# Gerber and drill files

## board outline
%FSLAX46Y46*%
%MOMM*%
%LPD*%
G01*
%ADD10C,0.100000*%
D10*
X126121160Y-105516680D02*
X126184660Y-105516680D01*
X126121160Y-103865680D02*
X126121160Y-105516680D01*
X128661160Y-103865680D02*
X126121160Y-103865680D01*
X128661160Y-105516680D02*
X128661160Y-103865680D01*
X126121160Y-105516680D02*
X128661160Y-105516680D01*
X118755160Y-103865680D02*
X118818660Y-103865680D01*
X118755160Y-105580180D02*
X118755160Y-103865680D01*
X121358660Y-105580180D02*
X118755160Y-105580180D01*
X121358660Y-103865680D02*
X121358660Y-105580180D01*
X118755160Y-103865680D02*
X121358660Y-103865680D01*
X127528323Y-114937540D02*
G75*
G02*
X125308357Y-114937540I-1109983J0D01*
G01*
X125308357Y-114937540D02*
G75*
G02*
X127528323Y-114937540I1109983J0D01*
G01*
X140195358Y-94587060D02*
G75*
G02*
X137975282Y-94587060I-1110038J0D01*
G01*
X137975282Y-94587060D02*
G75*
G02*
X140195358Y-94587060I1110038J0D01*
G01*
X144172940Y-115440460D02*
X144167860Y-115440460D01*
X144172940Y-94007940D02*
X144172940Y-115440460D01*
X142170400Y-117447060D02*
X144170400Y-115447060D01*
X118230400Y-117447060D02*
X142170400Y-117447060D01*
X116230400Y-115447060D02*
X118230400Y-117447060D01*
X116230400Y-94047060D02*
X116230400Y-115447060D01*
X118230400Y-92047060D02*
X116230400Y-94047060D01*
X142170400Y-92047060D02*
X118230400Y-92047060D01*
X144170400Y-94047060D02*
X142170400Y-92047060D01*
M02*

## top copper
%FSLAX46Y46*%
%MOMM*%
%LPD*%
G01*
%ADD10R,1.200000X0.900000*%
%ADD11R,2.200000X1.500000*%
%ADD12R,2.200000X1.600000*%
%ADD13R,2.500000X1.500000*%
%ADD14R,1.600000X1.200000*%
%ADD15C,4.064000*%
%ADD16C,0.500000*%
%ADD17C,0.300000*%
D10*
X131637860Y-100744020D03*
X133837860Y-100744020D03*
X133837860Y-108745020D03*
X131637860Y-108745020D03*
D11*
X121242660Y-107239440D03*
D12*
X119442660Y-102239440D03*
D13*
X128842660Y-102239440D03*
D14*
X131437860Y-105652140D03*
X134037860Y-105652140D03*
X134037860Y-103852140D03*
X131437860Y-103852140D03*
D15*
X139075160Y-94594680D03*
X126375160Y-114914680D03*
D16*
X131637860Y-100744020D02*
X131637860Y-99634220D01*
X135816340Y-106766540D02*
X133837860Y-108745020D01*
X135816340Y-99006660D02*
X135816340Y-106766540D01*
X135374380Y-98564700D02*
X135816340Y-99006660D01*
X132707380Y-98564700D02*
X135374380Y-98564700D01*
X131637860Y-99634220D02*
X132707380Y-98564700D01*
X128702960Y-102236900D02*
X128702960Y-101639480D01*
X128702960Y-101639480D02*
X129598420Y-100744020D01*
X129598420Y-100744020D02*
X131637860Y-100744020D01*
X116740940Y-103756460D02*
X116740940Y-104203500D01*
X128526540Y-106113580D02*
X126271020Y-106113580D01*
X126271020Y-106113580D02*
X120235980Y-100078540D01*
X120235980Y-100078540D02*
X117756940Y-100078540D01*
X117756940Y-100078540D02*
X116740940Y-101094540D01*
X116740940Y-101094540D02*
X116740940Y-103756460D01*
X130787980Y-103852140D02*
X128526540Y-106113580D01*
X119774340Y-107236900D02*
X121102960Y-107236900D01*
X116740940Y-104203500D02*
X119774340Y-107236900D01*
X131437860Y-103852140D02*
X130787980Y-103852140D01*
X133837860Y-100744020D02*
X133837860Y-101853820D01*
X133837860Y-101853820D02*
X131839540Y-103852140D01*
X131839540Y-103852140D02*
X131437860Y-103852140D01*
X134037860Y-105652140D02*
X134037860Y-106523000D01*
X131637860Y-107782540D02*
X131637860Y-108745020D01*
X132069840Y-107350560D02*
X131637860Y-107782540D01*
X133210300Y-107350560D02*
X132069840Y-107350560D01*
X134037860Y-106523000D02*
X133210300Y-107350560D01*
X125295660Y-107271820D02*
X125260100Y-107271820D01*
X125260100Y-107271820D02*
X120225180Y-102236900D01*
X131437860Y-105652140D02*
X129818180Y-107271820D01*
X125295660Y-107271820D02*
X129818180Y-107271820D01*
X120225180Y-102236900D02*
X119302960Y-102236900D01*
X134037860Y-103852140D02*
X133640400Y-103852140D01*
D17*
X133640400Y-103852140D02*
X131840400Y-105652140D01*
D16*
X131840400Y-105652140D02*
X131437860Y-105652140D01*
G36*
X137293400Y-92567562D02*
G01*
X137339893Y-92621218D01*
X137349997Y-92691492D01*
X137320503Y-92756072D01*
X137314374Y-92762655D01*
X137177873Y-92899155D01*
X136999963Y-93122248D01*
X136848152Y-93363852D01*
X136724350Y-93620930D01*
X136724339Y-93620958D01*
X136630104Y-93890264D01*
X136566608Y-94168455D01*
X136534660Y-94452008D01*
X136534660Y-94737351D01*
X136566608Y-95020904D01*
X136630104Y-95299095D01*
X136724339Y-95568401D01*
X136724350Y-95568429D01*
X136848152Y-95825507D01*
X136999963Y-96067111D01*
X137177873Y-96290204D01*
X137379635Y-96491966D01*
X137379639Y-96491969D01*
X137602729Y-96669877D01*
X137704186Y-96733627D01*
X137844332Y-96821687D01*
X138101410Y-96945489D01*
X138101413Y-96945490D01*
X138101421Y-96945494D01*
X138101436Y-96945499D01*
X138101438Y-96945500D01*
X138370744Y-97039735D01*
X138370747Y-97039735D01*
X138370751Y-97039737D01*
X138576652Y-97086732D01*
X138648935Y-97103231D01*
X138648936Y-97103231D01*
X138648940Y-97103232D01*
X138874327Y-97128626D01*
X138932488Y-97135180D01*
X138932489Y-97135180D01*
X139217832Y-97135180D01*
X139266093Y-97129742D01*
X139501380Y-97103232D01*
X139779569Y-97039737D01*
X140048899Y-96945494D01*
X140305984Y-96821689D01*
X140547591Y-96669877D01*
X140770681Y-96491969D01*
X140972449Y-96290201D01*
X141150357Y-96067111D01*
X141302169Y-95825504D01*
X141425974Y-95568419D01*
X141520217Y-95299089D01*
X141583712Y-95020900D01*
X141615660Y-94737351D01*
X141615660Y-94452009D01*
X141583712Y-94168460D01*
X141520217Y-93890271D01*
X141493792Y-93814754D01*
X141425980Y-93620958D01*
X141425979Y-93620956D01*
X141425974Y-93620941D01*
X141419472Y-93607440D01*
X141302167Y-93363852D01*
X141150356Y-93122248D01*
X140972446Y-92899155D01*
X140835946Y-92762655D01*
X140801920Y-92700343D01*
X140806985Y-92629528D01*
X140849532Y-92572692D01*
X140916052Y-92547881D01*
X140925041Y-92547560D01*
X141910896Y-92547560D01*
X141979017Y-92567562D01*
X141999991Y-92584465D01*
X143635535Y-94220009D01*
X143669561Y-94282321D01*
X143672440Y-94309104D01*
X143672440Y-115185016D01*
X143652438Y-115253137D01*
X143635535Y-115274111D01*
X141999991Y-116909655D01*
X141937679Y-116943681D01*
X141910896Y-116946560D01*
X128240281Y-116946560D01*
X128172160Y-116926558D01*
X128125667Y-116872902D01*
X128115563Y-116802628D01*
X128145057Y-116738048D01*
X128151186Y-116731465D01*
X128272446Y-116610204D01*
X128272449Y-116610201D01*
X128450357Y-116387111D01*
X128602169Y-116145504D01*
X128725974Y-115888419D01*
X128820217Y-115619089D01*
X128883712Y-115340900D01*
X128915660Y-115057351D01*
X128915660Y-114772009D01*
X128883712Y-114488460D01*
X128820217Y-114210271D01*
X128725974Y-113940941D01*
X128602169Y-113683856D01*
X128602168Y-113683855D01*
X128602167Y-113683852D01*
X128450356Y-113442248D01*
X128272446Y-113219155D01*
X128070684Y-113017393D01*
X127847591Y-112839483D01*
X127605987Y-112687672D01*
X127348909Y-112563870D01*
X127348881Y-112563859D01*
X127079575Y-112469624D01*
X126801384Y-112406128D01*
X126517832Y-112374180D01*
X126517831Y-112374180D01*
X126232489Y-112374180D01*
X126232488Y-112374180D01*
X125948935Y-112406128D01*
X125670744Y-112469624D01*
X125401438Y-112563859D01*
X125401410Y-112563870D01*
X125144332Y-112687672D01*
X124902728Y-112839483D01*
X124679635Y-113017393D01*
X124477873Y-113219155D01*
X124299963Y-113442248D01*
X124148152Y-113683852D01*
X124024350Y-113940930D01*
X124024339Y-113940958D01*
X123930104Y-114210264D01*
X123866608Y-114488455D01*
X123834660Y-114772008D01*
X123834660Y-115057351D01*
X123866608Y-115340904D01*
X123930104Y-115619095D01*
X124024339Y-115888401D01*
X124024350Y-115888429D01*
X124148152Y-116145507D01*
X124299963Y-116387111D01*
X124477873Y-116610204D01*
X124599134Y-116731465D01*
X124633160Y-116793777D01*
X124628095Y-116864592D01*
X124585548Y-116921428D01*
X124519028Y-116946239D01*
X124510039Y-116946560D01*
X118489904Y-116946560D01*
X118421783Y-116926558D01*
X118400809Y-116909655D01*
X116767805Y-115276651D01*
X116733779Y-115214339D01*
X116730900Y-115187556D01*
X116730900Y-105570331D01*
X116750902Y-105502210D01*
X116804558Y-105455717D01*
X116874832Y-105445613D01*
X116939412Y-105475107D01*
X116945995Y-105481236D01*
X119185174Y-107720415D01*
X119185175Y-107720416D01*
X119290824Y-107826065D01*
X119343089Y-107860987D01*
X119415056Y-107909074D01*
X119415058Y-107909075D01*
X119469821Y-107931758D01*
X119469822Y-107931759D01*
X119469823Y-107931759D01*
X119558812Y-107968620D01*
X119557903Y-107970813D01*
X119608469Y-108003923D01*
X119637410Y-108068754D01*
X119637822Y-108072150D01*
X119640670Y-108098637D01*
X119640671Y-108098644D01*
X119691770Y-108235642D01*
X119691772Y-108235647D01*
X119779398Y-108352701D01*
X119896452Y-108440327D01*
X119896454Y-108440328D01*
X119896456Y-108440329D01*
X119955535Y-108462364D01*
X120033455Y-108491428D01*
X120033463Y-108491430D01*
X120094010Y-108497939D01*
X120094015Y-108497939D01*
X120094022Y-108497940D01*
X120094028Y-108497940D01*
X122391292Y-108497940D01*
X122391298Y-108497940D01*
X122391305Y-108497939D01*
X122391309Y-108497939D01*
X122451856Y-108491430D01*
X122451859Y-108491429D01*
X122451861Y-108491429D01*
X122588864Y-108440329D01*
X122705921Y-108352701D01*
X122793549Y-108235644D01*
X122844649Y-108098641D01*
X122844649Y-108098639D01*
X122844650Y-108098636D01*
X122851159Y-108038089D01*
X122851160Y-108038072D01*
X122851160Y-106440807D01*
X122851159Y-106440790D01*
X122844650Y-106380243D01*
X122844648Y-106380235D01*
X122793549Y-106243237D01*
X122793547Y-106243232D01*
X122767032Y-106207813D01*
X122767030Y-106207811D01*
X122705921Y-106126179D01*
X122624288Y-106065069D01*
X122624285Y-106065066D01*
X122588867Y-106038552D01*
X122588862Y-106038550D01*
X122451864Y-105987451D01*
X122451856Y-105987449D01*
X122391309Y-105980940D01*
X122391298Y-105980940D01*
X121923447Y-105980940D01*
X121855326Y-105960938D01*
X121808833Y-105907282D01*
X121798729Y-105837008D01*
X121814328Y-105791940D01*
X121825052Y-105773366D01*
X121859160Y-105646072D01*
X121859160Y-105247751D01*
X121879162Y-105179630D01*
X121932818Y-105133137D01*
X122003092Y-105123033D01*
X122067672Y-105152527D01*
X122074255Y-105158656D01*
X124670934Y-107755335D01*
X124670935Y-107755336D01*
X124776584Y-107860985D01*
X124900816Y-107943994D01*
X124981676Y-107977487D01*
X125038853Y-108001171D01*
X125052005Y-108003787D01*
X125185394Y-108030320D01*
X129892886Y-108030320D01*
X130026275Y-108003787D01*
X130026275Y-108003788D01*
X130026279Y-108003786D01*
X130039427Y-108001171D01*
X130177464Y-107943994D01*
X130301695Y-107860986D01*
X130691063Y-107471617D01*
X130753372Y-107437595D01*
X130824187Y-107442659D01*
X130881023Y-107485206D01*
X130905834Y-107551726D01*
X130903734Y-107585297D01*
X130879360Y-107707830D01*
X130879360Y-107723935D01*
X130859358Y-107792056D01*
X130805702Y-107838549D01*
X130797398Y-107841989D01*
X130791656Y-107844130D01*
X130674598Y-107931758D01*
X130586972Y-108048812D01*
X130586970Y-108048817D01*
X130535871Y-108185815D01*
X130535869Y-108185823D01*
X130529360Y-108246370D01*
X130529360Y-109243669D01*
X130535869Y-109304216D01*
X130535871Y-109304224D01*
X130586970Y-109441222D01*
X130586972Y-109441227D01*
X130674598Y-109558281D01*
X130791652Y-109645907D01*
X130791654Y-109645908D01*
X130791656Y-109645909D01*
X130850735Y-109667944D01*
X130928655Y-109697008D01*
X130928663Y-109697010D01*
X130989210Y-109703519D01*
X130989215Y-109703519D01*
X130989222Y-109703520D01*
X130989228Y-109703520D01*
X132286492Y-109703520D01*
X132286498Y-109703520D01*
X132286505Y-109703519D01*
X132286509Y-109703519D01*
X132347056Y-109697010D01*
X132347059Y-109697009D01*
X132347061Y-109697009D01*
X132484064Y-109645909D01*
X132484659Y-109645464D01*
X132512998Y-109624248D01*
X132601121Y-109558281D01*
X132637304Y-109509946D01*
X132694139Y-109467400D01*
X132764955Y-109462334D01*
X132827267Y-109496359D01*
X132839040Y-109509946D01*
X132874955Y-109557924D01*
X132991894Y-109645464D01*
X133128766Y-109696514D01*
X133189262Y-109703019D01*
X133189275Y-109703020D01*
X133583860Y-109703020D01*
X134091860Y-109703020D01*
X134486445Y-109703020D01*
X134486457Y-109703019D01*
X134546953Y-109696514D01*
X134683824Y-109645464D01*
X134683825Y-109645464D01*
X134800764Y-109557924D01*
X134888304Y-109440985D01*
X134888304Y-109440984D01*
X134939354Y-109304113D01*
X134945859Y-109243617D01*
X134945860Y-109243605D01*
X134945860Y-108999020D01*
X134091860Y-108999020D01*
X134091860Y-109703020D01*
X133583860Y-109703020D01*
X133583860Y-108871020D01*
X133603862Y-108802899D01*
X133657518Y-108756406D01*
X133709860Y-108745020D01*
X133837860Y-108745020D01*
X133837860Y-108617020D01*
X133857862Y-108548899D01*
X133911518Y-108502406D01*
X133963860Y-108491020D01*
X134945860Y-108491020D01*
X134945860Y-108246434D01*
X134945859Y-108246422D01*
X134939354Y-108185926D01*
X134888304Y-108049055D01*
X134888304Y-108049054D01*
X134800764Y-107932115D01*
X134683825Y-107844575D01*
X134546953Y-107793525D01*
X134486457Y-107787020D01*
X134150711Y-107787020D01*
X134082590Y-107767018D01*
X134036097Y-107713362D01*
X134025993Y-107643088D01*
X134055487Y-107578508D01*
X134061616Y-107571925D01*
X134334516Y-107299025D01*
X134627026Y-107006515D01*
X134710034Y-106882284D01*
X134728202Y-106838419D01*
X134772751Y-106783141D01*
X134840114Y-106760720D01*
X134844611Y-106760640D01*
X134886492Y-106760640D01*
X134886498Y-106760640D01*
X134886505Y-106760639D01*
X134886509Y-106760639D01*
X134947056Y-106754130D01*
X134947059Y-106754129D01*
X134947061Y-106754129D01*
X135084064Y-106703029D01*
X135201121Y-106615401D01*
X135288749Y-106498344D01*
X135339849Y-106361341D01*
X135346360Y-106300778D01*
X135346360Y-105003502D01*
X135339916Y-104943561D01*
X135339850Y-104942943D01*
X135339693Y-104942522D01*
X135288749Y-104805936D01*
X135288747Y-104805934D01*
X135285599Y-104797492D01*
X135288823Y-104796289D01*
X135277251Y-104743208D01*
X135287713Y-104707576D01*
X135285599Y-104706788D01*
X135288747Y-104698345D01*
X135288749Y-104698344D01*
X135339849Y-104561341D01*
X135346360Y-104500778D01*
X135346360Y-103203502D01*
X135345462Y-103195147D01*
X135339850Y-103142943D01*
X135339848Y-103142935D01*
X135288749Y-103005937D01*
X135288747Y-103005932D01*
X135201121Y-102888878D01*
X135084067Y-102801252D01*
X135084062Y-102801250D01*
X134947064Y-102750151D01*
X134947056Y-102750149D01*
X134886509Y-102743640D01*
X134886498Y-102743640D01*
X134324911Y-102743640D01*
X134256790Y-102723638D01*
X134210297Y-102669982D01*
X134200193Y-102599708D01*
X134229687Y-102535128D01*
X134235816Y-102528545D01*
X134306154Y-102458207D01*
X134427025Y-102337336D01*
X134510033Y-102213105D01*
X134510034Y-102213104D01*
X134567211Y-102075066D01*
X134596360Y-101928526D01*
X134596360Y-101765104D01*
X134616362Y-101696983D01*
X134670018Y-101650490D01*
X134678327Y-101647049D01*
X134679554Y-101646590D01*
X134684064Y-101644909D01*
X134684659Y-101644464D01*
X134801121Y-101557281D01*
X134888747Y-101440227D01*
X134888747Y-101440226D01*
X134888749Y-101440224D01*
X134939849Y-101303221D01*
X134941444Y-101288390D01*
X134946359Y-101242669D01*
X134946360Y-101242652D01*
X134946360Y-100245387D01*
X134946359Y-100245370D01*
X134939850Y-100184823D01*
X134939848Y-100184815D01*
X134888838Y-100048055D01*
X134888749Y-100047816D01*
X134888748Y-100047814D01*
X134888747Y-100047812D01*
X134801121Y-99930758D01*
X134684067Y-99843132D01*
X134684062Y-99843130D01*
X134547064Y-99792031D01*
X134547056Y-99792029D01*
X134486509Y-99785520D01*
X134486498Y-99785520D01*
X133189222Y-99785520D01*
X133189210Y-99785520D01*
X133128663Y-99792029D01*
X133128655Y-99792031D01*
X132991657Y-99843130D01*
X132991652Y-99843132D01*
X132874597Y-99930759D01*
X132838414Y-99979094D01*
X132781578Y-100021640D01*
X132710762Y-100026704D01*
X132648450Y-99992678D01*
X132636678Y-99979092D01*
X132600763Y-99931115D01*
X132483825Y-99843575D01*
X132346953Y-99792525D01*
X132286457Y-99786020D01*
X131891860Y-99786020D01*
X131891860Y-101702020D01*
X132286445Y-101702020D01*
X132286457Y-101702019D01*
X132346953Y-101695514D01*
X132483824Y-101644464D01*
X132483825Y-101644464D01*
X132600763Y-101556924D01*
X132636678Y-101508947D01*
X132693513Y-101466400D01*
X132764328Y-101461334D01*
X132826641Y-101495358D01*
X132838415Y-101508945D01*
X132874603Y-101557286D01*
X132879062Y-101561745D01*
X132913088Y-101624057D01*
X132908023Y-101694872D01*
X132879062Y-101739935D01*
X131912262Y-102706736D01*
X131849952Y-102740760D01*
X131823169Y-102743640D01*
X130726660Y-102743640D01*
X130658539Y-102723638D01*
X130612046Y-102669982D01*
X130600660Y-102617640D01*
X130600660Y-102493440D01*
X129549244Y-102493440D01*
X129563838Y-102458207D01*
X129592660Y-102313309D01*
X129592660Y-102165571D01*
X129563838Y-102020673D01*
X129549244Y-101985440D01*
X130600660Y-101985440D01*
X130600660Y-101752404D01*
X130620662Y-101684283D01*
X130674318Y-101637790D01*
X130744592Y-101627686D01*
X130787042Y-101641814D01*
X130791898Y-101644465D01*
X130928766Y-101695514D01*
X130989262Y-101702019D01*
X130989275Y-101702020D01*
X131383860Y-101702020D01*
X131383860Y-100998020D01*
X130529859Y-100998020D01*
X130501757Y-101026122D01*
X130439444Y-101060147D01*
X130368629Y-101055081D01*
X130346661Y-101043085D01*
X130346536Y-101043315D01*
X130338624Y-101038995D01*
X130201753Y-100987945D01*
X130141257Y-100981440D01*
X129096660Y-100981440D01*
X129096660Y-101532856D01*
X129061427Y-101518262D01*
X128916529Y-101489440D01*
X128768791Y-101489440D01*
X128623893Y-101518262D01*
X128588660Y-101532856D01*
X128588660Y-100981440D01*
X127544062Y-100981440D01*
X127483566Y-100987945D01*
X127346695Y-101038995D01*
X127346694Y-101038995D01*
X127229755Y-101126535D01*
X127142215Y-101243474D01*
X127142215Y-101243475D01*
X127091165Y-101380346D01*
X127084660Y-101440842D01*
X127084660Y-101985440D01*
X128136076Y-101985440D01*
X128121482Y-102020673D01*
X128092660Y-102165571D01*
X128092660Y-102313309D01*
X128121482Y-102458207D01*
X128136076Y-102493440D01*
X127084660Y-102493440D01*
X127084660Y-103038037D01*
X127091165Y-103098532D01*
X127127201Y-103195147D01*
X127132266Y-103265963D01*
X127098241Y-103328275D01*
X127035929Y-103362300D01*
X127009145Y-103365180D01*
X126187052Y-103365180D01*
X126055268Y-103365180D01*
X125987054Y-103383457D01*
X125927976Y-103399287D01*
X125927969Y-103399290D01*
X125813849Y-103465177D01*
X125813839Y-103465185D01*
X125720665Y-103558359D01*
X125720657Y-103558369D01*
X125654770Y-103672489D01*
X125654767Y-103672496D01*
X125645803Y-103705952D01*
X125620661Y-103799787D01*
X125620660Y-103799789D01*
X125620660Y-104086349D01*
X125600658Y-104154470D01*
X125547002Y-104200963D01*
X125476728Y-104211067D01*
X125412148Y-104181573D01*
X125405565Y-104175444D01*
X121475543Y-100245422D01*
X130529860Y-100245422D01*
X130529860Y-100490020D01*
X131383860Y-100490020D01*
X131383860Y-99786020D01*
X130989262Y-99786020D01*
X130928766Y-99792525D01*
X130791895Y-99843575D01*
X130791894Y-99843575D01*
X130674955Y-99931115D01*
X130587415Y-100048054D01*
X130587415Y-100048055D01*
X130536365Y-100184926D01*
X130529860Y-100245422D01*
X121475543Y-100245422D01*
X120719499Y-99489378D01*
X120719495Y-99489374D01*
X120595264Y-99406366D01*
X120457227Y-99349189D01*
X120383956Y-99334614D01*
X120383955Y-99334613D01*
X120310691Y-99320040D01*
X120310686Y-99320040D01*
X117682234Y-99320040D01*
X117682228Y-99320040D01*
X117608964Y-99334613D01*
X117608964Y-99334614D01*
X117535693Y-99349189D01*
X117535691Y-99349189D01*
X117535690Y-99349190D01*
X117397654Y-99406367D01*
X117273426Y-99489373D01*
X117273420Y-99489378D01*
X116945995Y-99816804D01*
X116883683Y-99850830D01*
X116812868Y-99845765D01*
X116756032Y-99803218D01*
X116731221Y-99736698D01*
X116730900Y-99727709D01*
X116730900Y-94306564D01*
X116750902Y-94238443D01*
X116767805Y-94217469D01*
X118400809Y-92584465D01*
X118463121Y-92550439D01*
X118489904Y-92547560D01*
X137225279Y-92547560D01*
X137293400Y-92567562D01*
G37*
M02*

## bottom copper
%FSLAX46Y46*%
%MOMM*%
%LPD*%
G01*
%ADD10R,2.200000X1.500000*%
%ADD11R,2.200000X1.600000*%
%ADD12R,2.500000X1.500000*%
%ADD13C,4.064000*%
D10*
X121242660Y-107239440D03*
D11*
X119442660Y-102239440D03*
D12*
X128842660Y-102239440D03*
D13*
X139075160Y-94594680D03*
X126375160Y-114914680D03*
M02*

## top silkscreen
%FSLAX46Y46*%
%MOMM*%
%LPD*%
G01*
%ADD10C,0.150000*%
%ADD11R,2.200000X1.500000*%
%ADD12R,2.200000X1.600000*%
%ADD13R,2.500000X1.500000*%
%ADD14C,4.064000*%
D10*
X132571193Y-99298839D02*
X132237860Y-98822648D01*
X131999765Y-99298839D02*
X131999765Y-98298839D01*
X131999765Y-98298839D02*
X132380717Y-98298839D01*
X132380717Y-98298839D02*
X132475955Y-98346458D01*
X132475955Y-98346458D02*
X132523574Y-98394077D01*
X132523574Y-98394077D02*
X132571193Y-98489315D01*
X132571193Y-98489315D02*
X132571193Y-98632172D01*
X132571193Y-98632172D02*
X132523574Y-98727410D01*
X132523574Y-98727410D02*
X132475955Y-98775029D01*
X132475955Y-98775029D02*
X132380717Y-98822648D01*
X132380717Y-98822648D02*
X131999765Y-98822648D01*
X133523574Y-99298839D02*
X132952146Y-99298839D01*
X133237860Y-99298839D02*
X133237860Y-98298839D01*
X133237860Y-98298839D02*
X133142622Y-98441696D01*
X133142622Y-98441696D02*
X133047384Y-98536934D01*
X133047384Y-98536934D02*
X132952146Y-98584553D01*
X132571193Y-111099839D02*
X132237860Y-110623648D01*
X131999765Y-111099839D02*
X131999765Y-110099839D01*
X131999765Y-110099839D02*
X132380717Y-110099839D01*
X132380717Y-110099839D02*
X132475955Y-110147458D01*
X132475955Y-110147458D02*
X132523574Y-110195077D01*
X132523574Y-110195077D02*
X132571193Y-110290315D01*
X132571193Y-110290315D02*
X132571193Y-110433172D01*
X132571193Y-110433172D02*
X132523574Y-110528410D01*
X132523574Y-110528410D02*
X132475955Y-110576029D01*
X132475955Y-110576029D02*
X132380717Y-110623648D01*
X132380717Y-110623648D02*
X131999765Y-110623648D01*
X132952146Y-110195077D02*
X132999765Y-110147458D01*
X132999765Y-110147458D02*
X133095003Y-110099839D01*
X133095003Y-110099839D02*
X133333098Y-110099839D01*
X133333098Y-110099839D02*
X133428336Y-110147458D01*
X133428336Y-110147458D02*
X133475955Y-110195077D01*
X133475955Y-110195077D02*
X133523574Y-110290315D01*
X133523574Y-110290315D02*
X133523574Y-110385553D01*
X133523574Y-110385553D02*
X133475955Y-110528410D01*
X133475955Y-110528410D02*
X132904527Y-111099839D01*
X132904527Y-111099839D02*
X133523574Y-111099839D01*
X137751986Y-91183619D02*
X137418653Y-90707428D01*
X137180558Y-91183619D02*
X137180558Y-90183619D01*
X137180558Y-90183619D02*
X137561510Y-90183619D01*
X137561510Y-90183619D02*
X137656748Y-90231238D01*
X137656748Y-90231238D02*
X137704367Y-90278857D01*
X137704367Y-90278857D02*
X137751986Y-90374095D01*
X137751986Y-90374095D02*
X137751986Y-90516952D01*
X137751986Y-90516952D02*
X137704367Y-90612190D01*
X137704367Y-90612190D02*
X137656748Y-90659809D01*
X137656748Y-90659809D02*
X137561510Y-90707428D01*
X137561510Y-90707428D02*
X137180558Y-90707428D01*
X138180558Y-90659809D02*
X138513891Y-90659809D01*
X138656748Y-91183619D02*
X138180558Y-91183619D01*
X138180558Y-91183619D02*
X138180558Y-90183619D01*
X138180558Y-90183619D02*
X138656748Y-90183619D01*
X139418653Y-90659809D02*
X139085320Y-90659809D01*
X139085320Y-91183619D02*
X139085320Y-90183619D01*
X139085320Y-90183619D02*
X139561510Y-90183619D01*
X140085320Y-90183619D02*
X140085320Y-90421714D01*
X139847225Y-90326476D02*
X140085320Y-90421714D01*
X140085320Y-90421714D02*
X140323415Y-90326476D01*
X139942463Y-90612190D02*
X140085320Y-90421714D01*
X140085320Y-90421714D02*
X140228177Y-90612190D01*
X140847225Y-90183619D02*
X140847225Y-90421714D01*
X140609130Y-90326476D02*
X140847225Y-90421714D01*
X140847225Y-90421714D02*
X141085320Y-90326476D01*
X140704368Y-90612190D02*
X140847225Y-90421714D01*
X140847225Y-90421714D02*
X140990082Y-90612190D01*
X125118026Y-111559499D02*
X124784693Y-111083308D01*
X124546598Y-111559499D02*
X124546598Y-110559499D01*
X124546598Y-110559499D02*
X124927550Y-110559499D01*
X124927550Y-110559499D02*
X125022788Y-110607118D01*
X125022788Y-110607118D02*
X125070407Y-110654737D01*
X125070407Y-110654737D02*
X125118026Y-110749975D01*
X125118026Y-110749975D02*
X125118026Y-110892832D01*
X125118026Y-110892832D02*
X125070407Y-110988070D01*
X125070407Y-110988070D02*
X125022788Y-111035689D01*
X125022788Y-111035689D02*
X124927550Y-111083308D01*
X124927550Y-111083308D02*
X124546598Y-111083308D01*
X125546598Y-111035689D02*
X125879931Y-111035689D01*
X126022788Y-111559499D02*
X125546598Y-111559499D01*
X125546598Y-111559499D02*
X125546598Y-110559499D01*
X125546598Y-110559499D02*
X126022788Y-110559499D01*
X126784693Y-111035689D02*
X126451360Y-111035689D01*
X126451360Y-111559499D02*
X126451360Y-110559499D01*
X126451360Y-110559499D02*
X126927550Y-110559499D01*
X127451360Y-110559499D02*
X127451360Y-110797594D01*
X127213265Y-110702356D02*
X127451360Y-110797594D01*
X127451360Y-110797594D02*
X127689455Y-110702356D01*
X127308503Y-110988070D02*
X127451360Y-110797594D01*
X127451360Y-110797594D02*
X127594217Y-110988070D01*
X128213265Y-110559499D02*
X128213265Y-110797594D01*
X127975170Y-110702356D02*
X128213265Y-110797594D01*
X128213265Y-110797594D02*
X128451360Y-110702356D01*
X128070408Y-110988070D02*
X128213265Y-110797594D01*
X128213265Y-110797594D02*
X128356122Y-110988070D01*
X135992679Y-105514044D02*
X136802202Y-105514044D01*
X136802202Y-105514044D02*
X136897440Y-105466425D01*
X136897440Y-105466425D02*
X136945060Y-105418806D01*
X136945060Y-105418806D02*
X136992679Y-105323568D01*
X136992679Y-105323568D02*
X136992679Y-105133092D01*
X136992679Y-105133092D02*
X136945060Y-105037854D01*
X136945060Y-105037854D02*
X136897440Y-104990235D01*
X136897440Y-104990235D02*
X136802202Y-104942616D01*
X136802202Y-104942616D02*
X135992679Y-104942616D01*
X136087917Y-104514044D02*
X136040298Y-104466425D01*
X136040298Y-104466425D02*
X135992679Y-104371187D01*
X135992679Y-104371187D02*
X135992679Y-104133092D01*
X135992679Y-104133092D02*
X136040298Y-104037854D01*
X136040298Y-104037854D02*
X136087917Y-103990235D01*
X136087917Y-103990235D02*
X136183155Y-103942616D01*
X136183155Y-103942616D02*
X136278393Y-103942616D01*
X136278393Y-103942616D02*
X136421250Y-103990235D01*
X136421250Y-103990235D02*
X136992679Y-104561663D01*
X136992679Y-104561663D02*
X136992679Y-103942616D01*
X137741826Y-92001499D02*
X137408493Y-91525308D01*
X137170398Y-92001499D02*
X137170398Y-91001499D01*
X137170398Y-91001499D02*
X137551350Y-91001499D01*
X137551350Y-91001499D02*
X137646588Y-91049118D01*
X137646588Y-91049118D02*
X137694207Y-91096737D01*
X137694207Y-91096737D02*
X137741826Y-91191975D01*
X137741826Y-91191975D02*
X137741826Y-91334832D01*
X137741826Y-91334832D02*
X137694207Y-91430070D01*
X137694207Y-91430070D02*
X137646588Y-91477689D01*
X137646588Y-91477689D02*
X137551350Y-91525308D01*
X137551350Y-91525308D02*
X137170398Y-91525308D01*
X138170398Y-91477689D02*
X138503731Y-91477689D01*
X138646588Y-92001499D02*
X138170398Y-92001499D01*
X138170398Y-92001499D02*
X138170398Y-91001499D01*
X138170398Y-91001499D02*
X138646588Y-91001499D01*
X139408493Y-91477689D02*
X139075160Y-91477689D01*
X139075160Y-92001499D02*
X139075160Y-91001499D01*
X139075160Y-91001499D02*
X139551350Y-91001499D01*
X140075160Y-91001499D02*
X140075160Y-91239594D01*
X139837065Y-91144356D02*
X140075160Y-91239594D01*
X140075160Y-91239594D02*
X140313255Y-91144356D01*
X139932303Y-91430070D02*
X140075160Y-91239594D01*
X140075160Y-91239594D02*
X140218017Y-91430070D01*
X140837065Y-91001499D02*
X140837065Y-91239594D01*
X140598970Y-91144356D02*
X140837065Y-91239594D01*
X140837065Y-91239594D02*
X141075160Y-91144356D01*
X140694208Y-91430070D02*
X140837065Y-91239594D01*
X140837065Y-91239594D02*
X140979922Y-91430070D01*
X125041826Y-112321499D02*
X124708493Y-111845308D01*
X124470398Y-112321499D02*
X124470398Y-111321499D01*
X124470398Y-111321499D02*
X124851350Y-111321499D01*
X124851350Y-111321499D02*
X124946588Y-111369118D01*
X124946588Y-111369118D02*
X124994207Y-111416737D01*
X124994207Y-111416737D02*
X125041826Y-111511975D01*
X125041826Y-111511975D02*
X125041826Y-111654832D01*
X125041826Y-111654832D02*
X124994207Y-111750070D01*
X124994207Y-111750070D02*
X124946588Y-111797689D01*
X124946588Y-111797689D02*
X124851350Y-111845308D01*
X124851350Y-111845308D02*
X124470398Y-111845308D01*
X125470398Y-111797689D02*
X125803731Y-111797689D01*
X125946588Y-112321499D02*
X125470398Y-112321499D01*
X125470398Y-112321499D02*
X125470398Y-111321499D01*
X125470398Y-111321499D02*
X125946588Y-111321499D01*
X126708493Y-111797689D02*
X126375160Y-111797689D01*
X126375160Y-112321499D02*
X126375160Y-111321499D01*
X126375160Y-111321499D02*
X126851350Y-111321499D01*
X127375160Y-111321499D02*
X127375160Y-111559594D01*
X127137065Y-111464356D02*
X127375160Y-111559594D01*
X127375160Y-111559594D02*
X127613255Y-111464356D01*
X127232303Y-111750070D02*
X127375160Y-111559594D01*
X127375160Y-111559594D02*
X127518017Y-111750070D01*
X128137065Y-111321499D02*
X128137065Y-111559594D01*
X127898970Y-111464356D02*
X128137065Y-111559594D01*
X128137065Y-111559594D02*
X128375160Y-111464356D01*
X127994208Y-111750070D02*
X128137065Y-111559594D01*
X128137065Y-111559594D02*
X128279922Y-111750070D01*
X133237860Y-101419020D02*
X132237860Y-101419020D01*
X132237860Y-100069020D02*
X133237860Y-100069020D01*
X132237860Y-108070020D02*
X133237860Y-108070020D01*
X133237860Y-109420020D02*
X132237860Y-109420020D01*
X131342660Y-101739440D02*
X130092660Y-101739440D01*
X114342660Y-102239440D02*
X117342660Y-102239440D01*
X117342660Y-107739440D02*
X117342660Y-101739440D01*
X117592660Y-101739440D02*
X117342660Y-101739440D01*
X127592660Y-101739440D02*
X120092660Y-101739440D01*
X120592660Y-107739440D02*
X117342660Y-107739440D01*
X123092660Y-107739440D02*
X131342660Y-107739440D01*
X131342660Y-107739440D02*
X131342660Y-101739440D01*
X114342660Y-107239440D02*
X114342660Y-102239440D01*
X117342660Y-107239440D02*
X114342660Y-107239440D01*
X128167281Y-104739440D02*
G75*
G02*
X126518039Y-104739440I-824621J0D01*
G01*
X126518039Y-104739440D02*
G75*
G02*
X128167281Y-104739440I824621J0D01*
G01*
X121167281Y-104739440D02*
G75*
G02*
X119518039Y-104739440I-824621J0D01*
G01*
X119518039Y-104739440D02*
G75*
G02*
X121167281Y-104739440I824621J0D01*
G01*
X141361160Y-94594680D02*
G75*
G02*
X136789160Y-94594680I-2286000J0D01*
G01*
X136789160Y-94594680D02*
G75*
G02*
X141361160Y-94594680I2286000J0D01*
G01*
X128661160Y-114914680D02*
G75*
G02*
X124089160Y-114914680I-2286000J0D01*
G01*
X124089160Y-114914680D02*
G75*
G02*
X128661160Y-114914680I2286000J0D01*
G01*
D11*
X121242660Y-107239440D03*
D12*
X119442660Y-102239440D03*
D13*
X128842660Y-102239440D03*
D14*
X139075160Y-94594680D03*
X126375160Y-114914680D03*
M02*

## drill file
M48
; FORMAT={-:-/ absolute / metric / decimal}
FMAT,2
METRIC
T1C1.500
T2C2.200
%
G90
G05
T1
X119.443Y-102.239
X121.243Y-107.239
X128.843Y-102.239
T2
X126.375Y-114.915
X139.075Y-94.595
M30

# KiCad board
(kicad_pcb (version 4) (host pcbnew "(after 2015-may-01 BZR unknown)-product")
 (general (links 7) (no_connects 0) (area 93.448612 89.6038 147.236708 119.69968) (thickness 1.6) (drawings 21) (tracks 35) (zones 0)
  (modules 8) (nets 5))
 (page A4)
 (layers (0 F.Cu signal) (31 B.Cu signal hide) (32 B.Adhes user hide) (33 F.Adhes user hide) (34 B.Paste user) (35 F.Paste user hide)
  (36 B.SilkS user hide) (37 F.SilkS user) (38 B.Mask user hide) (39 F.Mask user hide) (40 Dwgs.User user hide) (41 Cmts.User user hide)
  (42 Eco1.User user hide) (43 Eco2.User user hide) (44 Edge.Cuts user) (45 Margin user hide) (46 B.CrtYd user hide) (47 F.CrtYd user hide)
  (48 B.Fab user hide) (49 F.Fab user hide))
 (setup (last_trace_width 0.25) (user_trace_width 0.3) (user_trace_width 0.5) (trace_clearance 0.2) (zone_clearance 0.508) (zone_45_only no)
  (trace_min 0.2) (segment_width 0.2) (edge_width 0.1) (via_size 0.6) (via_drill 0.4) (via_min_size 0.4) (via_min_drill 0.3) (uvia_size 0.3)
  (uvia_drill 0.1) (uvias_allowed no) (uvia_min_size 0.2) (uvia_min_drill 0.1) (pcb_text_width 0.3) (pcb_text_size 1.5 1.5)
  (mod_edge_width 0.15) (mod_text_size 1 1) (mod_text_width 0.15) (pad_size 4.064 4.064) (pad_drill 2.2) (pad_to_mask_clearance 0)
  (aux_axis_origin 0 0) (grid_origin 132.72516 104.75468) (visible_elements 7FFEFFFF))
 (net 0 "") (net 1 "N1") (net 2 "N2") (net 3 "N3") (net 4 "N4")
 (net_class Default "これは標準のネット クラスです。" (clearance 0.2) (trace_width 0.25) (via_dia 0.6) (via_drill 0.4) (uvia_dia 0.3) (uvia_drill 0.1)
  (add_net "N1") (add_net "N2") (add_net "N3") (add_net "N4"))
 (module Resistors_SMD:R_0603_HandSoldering (layer F.Cu) (at 132.73786 100.74402)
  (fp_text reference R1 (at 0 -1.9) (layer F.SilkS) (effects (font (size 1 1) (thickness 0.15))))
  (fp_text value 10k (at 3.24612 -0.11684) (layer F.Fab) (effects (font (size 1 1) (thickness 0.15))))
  (fp_line (start 0.5 0.675) (end -0.5 0.675) (layer F.SilkS) (width 0.15))
  (fp_line (start -0.5 -0.675) (end 0.5 -0.675) (layer F.SilkS) (width 0.15))
  (pad 1 smd rect (at -1.1 0) (size 1.2 0.9) (layers F.Cu F.Paste F.Mask) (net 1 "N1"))
  (pad 2 smd rect (at 1.1 0) (size 1.2 0.9) (layers F.Cu F.Paste F.Mask) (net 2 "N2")))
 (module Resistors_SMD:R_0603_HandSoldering (layer F.Cu) (at 132.73786 108.74502 180)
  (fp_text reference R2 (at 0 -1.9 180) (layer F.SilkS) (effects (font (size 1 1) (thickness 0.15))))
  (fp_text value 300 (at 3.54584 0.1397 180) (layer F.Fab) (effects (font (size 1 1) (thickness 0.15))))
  (fp_line (start 0.5 0.675) (end -0.5 0.675) (layer F.SilkS) (width 0.15))
  (fp_line (start -0.5 -0.675) (end 0.5 -0.675) (layer F.SilkS) (width 0.15))
  (pad 1 smd rect (at -1.1 0 180) (size 1.2 0.9) (layers F.Cu F.Paste F.Mask) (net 1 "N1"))
  (pad 2 smd rect (at 1.1 0 180) (size 1.2 0.9) (layers F.Cu F.Paste F.Mask) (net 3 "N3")))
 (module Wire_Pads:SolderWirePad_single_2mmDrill (layer F.Cu) (at 139.08532 94.5388)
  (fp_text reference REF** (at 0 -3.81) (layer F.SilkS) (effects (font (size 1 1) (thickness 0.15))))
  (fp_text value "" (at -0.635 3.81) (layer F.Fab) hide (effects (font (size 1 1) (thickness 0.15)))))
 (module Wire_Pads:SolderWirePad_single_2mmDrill (layer F.Cu) (at 126.45136 114.91468)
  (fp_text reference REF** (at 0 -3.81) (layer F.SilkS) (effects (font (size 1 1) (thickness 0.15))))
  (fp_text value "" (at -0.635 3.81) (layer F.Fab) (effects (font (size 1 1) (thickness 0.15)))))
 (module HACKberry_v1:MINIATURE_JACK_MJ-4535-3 (layer F.Cu) (at 120.34266 104.73944 180)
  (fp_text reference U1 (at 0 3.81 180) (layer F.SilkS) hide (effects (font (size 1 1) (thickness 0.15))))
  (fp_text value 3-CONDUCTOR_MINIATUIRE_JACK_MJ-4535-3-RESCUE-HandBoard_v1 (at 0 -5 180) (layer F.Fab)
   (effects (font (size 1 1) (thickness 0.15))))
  (fp_line (start -11 3) (end -9.75 3) (layer F.SilkS) (width 0.15))
  (fp_line (start 6 2.5) (end 3 2.5) (layer F.SilkS) (width 0.15))
  (fp_line (start 3 -3) (end 3 3) (layer F.SilkS) (width 0.15))
  (fp_line (start 2.75 3) (end 3 3) (layer F.SilkS) (width 0.15))
  (fp_line (start -7.25 3) (end 0.25 3) (layer F.SilkS) (width 0.15))
  (fp_line (start -0.25 -3) (end 3 -3) (layer F.SilkS) (width 0.15))
  (fp_line (start -2.75 -3) (end -11 -3) (layer F.SilkS) (width 0.15))
  (fp_line (start -11 -3) (end -11 3) (layer F.SilkS) (width 0.15))
  (fp_line (start 6 -2.5) (end 6 2.5) (layer F.SilkS) (width 0.15))
  (fp_line (start 3 -2.5) (end 6 -2.5) (layer F.SilkS) (width 0.15))
  (fp_circle (center -7 0) (end -6.8 0.8) (layer F.SilkS) (width 0.15))
  (fp_circle (center 0 0) (end -0.2 0.8) (layer F.SilkS) (width 0.15))
  (pad 4 thru_hole rect (at -0.9 -2.5 180) (size 2.2 1.5) (drill 1.5) (layers *.Cu *.Mask F.SilkS) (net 2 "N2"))
  (pad 2 thru_hole rect (at 0.9 2.5 180) (size 2.2 1.6) (drill 1.5) (layers *.Cu *.Mask F.SilkS) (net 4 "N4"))
  (pad 1 thru_hole rect (at -8.5 2.5 180) (size 2.5 1.5) (drill 1.5) (layers *.Cu *.Mask F.SilkS) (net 1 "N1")))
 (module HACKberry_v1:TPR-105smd (layer F.Cu) (at 132.73786 104.75214 90)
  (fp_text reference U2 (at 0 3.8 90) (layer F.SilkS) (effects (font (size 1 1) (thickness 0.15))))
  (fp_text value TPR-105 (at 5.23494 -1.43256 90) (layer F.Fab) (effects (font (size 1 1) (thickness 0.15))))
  (pad 1 smd rect (at -0.9 -1.3 90) (size 1.2 1.6) (layers F.Cu F.Paste F.Mask) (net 4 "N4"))
  (pad 2 smd rect (at -0.9 1.3 90) (size 1.2 1.6) (layers F.Cu F.Paste F.Mask) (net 3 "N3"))
  (pad 3 smd rect (at 0.9 1.3 90) (size 1.2 1.6) (layers F.Cu F.Paste F.Mask) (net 4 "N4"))
  (pad 4 smd rect (at 0.9 -1.3 90) (size 1.2 1.6) (layers F.Cu F.Paste F.Mask) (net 2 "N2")))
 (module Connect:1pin (layer F.Cu) (at 139.07516 94.59468)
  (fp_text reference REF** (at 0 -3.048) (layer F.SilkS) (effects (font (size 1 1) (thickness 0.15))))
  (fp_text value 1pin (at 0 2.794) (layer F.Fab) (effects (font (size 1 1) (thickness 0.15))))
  (fp_circle (center 0 0) (end 0 -2.286) (layer F.SilkS) (width 0.15))
  (pad 1 thru_hole circle (at 0 0) (size 4.064 4.064) (drill 2.2) (layers *.Cu *.Mask F.SilkS)))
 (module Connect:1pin (layer F.Cu) (at 126.37516 114.91468)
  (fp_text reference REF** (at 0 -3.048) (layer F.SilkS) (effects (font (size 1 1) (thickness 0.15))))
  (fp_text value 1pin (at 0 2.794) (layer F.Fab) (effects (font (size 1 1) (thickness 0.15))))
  (fp_circle (center 0 0) (end 0 -2.286) (layer F.SilkS) (width 0.15))
  (pad 1 thru_hole circle (at 0 0) (size 4.064 4.064) (drill 2.2) (layers *.Cu *.Mask F.SilkS)))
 (gr_line (start 126.12116 105.51668) (end 126.18466 105.51668) (angle 90) (layer Edge.Cuts) (width 0.1))
 (gr_line (start 126.12116 103.86568) (end 126.12116 105.51668) (angle 90) (layer Edge.Cuts) (width 0.1))
 (gr_line (start 128.66116 103.86568) (end 126.12116 103.86568) (angle 90) (layer Edge.Cuts) (width 0.1))
 (gr_line (start 128.66116 105.51668) (end 128.66116 103.86568) (angle 90) (layer Edge.Cuts) (width 0.1))
 (gr_line (start 126.12116 105.51668) (end 128.66116 105.51668) (angle 90) (layer Edge.Cuts) (width 0.1))
 (gr_line (start 118.75516 103.86568) (end 118.81866 103.86568) (angle 90) (layer Edge.Cuts) (width 0.1))
 (gr_line (start 118.75516 105.58018) (end 118.75516 103.86568) (angle 90) (layer Edge.Cuts) (width 0.1))
 (gr_line (start 121.35866 105.58018) (end 118.75516 105.58018) (angle 90) (layer Edge.Cuts) (width 0.1))
 (gr_line (start 121.35866 103.86568) (end 121.35866 105.58018) (angle 90) (layer Edge.Cuts) (width 0.1))
 (gr_line (start 118.75516 103.86568) (end 121.35866 103.86568) (angle 90) (layer Edge.Cuts) (width 0.1))
 (gr_circle (center 126.41834 114.93754) (end 126.42088 113.82756) (layer Edge.Cuts) (width 0.1))
 (gr_circle (center 139.08532 94.58706) (end 139.192 93.48216) (layer Edge.Cuts) (width 0.1))
 (gr_line (start 144.17294 115.44046) (end 144.16786 115.44046) (angle 90) (layer Edge.Cuts) (width 0.1))
 (gr_line (start 144.17294 94.00794) (end 144.17294 115.44046) (angle 90) (layer Edge.Cuts) (width 0.1))
 (gr_line (start 142.1704 117.44706) (end 144.1704 115.44706) (layer Edge.Cuts) (width 0.1))
 (gr_line (start 118.2304 117.44706) (end 142.1704 117.44706) (layer Edge.Cuts) (width 0.1))
 (gr_line (start 116.2304 115.44706) (end 118.2304 117.44706) (layer Edge.Cuts) (width 0.1))
 (gr_line (start 116.2304 94.04706) (end 116.2304 115.44706) (layer Edge.Cuts) (width 0.1))
 (gr_line (start 118.2304 92.04706) (end 116.2304 94.04706) (layer Edge.Cuts) (width 0.1))
 (gr_line (start 142.1704 92.04706) (end 118.2304 92.04706) (layer Edge.Cuts) (width 0.1))
 (gr_line (start 144.1704 94.04706) (end 142.1704 92.04706) (layer Edge.Cuts) (width 0.1))
 (segment (start 131.63786 100.74402) (end 131.63786 99.63422) (width 0.5) (layer F.Cu) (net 1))
 (segment (start 135.81634 106.76654) (end 133.83786 108.74502) (width 0.5) (layer F.Cu) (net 1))
 (segment (start 135.81634 99.00666) (end 135.81634 106.76654) (width 0.5) (layer F.Cu) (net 1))
 (segment (start 135.37438 98.5647) (end 135.81634 99.00666) (width 0.5) (layer F.Cu) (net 1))
 (segment (start 132.70738 98.5647) (end 135.37438 98.5647) (width 0.5) (layer F.Cu) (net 1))
 (segment (start 131.63786 99.63422) (end 132.70738 98.5647) (width 0.5) (layer F.Cu) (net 1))
 (segment (start 128.70296 102.2369) (end 128.70296 101.63948) (width 0.5) (layer F.Cu) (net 1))
 (segment (start 128.70296 101.63948) (end 129.59842 100.74402) (width 0.5) (layer F.Cu) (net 1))
 (segment (start 129.59842 100.74402) (end 131.63786 100.74402) (width 0.5) (layer F.Cu) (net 1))
 (segment (start 116.74094 103.75646) (end 116.74094 104.2035) (width 0.5) (layer F.Cu) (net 2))
 (segment (start 128.52654 106.11358) (end 126.27102 106.11358) (width 0.5) (layer F.Cu) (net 2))
 (segment (start 126.27102 106.11358) (end 120.23598 100.07854) (width 0.5) (layer F.Cu) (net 2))
 (segment (start 120.23598 100.07854) (end 117.75694 100.07854) (width 0.5) (layer F.Cu) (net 2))
 (segment (start 117.75694 100.07854) (end 116.74094 101.09454) (width 0.5) (layer F.Cu) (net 2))
 (segment (start 116.74094 101.09454) (end 116.74094 103.75646) (width 0.5) (layer F.Cu) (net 2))
 (segment (start 130.78798 103.85214) (end 128.52654 106.11358) (width 0.5) (layer F.Cu) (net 2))
 (segment (start 119.77434 107.2369) (end 121.10296 107.2369) (width 0.5) (layer F.Cu) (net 2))
 (segment (start 116.74094 104.2035) (end 119.77434 107.2369) (width 0.5) (layer F.Cu) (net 2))
 (segment (start 131.43786 103.85214) (end 130.78798 103.85214) (width 0.5) (layer F.Cu) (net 2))
 (segment (start 133.83786 100.74402) (end 133.83786 101.85382) (width 0.5) (layer F.Cu) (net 2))
 (segment (start 133.83786 101.85382) (end 131.83954 103.85214) (width 0.5) (layer F.Cu) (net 2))
 (segment (start 131.83954 103.85214) (end 131.43786 103.85214) (width 0.5) (layer F.Cu) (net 2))
 (segment (start 134.03786 105.65214) (end 134.03786 106.523) (width 0.5) (layer F.Cu) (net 3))
 (segment (start 131.63786 107.78254) (end 131.63786 108.74502) (width 0.5) (layer F.Cu) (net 3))
 (segment (start 132.06984 107.35056) (end 131.63786 107.78254) (width 0.5) (layer F.Cu) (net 3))
 (segment (start 133.2103 107.35056) (end 132.06984 107.35056) (width 0.5) (layer F.Cu) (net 3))
 (segment (start 134.03786 106.523) (end 133.2103 107.35056) (width 0.5) (layer F.Cu) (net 3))
 (segment (start 125.29566 107.27182) (end 125.2601 107.27182) (width 0.5) (layer F.Cu) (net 4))
 (segment (start 125.2601 107.27182) (end 120.22518 102.2369) (width 0.5) (layer F.Cu) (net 4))
 (segment (start 131.43786 105.65214) (end 129.81818 107.27182) (width 0.5) (layer F.Cu) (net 4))
 (segment (start 125.29566 107.27182) (end 129.81818 107.27182) (width 0.5) (layer F.Cu) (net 4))
 (segment (start 120.22518 102.2369) (end 119.30296 102.2369) (width 0.5) (layer F.Cu) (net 4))
 (segment (start 134.03786 103.85214) (end 133.6404 103.85214) (width 0.5) (layer F.Cu) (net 4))
 (segment (start 133.6404 103.85214) (end 131.8404 105.65214) (width 0.3) (layer F.Cu) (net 4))
 (segment (start 131.8404 105.65214) (end 131.43786 105.65214) (width 0.5) (layer F.Cu) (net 4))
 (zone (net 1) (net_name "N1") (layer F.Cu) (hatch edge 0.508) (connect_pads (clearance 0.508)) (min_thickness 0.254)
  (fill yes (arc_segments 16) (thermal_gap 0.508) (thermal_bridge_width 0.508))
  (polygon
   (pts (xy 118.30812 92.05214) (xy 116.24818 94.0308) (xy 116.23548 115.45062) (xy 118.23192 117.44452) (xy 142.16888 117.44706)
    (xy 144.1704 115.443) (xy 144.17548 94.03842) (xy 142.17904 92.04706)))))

